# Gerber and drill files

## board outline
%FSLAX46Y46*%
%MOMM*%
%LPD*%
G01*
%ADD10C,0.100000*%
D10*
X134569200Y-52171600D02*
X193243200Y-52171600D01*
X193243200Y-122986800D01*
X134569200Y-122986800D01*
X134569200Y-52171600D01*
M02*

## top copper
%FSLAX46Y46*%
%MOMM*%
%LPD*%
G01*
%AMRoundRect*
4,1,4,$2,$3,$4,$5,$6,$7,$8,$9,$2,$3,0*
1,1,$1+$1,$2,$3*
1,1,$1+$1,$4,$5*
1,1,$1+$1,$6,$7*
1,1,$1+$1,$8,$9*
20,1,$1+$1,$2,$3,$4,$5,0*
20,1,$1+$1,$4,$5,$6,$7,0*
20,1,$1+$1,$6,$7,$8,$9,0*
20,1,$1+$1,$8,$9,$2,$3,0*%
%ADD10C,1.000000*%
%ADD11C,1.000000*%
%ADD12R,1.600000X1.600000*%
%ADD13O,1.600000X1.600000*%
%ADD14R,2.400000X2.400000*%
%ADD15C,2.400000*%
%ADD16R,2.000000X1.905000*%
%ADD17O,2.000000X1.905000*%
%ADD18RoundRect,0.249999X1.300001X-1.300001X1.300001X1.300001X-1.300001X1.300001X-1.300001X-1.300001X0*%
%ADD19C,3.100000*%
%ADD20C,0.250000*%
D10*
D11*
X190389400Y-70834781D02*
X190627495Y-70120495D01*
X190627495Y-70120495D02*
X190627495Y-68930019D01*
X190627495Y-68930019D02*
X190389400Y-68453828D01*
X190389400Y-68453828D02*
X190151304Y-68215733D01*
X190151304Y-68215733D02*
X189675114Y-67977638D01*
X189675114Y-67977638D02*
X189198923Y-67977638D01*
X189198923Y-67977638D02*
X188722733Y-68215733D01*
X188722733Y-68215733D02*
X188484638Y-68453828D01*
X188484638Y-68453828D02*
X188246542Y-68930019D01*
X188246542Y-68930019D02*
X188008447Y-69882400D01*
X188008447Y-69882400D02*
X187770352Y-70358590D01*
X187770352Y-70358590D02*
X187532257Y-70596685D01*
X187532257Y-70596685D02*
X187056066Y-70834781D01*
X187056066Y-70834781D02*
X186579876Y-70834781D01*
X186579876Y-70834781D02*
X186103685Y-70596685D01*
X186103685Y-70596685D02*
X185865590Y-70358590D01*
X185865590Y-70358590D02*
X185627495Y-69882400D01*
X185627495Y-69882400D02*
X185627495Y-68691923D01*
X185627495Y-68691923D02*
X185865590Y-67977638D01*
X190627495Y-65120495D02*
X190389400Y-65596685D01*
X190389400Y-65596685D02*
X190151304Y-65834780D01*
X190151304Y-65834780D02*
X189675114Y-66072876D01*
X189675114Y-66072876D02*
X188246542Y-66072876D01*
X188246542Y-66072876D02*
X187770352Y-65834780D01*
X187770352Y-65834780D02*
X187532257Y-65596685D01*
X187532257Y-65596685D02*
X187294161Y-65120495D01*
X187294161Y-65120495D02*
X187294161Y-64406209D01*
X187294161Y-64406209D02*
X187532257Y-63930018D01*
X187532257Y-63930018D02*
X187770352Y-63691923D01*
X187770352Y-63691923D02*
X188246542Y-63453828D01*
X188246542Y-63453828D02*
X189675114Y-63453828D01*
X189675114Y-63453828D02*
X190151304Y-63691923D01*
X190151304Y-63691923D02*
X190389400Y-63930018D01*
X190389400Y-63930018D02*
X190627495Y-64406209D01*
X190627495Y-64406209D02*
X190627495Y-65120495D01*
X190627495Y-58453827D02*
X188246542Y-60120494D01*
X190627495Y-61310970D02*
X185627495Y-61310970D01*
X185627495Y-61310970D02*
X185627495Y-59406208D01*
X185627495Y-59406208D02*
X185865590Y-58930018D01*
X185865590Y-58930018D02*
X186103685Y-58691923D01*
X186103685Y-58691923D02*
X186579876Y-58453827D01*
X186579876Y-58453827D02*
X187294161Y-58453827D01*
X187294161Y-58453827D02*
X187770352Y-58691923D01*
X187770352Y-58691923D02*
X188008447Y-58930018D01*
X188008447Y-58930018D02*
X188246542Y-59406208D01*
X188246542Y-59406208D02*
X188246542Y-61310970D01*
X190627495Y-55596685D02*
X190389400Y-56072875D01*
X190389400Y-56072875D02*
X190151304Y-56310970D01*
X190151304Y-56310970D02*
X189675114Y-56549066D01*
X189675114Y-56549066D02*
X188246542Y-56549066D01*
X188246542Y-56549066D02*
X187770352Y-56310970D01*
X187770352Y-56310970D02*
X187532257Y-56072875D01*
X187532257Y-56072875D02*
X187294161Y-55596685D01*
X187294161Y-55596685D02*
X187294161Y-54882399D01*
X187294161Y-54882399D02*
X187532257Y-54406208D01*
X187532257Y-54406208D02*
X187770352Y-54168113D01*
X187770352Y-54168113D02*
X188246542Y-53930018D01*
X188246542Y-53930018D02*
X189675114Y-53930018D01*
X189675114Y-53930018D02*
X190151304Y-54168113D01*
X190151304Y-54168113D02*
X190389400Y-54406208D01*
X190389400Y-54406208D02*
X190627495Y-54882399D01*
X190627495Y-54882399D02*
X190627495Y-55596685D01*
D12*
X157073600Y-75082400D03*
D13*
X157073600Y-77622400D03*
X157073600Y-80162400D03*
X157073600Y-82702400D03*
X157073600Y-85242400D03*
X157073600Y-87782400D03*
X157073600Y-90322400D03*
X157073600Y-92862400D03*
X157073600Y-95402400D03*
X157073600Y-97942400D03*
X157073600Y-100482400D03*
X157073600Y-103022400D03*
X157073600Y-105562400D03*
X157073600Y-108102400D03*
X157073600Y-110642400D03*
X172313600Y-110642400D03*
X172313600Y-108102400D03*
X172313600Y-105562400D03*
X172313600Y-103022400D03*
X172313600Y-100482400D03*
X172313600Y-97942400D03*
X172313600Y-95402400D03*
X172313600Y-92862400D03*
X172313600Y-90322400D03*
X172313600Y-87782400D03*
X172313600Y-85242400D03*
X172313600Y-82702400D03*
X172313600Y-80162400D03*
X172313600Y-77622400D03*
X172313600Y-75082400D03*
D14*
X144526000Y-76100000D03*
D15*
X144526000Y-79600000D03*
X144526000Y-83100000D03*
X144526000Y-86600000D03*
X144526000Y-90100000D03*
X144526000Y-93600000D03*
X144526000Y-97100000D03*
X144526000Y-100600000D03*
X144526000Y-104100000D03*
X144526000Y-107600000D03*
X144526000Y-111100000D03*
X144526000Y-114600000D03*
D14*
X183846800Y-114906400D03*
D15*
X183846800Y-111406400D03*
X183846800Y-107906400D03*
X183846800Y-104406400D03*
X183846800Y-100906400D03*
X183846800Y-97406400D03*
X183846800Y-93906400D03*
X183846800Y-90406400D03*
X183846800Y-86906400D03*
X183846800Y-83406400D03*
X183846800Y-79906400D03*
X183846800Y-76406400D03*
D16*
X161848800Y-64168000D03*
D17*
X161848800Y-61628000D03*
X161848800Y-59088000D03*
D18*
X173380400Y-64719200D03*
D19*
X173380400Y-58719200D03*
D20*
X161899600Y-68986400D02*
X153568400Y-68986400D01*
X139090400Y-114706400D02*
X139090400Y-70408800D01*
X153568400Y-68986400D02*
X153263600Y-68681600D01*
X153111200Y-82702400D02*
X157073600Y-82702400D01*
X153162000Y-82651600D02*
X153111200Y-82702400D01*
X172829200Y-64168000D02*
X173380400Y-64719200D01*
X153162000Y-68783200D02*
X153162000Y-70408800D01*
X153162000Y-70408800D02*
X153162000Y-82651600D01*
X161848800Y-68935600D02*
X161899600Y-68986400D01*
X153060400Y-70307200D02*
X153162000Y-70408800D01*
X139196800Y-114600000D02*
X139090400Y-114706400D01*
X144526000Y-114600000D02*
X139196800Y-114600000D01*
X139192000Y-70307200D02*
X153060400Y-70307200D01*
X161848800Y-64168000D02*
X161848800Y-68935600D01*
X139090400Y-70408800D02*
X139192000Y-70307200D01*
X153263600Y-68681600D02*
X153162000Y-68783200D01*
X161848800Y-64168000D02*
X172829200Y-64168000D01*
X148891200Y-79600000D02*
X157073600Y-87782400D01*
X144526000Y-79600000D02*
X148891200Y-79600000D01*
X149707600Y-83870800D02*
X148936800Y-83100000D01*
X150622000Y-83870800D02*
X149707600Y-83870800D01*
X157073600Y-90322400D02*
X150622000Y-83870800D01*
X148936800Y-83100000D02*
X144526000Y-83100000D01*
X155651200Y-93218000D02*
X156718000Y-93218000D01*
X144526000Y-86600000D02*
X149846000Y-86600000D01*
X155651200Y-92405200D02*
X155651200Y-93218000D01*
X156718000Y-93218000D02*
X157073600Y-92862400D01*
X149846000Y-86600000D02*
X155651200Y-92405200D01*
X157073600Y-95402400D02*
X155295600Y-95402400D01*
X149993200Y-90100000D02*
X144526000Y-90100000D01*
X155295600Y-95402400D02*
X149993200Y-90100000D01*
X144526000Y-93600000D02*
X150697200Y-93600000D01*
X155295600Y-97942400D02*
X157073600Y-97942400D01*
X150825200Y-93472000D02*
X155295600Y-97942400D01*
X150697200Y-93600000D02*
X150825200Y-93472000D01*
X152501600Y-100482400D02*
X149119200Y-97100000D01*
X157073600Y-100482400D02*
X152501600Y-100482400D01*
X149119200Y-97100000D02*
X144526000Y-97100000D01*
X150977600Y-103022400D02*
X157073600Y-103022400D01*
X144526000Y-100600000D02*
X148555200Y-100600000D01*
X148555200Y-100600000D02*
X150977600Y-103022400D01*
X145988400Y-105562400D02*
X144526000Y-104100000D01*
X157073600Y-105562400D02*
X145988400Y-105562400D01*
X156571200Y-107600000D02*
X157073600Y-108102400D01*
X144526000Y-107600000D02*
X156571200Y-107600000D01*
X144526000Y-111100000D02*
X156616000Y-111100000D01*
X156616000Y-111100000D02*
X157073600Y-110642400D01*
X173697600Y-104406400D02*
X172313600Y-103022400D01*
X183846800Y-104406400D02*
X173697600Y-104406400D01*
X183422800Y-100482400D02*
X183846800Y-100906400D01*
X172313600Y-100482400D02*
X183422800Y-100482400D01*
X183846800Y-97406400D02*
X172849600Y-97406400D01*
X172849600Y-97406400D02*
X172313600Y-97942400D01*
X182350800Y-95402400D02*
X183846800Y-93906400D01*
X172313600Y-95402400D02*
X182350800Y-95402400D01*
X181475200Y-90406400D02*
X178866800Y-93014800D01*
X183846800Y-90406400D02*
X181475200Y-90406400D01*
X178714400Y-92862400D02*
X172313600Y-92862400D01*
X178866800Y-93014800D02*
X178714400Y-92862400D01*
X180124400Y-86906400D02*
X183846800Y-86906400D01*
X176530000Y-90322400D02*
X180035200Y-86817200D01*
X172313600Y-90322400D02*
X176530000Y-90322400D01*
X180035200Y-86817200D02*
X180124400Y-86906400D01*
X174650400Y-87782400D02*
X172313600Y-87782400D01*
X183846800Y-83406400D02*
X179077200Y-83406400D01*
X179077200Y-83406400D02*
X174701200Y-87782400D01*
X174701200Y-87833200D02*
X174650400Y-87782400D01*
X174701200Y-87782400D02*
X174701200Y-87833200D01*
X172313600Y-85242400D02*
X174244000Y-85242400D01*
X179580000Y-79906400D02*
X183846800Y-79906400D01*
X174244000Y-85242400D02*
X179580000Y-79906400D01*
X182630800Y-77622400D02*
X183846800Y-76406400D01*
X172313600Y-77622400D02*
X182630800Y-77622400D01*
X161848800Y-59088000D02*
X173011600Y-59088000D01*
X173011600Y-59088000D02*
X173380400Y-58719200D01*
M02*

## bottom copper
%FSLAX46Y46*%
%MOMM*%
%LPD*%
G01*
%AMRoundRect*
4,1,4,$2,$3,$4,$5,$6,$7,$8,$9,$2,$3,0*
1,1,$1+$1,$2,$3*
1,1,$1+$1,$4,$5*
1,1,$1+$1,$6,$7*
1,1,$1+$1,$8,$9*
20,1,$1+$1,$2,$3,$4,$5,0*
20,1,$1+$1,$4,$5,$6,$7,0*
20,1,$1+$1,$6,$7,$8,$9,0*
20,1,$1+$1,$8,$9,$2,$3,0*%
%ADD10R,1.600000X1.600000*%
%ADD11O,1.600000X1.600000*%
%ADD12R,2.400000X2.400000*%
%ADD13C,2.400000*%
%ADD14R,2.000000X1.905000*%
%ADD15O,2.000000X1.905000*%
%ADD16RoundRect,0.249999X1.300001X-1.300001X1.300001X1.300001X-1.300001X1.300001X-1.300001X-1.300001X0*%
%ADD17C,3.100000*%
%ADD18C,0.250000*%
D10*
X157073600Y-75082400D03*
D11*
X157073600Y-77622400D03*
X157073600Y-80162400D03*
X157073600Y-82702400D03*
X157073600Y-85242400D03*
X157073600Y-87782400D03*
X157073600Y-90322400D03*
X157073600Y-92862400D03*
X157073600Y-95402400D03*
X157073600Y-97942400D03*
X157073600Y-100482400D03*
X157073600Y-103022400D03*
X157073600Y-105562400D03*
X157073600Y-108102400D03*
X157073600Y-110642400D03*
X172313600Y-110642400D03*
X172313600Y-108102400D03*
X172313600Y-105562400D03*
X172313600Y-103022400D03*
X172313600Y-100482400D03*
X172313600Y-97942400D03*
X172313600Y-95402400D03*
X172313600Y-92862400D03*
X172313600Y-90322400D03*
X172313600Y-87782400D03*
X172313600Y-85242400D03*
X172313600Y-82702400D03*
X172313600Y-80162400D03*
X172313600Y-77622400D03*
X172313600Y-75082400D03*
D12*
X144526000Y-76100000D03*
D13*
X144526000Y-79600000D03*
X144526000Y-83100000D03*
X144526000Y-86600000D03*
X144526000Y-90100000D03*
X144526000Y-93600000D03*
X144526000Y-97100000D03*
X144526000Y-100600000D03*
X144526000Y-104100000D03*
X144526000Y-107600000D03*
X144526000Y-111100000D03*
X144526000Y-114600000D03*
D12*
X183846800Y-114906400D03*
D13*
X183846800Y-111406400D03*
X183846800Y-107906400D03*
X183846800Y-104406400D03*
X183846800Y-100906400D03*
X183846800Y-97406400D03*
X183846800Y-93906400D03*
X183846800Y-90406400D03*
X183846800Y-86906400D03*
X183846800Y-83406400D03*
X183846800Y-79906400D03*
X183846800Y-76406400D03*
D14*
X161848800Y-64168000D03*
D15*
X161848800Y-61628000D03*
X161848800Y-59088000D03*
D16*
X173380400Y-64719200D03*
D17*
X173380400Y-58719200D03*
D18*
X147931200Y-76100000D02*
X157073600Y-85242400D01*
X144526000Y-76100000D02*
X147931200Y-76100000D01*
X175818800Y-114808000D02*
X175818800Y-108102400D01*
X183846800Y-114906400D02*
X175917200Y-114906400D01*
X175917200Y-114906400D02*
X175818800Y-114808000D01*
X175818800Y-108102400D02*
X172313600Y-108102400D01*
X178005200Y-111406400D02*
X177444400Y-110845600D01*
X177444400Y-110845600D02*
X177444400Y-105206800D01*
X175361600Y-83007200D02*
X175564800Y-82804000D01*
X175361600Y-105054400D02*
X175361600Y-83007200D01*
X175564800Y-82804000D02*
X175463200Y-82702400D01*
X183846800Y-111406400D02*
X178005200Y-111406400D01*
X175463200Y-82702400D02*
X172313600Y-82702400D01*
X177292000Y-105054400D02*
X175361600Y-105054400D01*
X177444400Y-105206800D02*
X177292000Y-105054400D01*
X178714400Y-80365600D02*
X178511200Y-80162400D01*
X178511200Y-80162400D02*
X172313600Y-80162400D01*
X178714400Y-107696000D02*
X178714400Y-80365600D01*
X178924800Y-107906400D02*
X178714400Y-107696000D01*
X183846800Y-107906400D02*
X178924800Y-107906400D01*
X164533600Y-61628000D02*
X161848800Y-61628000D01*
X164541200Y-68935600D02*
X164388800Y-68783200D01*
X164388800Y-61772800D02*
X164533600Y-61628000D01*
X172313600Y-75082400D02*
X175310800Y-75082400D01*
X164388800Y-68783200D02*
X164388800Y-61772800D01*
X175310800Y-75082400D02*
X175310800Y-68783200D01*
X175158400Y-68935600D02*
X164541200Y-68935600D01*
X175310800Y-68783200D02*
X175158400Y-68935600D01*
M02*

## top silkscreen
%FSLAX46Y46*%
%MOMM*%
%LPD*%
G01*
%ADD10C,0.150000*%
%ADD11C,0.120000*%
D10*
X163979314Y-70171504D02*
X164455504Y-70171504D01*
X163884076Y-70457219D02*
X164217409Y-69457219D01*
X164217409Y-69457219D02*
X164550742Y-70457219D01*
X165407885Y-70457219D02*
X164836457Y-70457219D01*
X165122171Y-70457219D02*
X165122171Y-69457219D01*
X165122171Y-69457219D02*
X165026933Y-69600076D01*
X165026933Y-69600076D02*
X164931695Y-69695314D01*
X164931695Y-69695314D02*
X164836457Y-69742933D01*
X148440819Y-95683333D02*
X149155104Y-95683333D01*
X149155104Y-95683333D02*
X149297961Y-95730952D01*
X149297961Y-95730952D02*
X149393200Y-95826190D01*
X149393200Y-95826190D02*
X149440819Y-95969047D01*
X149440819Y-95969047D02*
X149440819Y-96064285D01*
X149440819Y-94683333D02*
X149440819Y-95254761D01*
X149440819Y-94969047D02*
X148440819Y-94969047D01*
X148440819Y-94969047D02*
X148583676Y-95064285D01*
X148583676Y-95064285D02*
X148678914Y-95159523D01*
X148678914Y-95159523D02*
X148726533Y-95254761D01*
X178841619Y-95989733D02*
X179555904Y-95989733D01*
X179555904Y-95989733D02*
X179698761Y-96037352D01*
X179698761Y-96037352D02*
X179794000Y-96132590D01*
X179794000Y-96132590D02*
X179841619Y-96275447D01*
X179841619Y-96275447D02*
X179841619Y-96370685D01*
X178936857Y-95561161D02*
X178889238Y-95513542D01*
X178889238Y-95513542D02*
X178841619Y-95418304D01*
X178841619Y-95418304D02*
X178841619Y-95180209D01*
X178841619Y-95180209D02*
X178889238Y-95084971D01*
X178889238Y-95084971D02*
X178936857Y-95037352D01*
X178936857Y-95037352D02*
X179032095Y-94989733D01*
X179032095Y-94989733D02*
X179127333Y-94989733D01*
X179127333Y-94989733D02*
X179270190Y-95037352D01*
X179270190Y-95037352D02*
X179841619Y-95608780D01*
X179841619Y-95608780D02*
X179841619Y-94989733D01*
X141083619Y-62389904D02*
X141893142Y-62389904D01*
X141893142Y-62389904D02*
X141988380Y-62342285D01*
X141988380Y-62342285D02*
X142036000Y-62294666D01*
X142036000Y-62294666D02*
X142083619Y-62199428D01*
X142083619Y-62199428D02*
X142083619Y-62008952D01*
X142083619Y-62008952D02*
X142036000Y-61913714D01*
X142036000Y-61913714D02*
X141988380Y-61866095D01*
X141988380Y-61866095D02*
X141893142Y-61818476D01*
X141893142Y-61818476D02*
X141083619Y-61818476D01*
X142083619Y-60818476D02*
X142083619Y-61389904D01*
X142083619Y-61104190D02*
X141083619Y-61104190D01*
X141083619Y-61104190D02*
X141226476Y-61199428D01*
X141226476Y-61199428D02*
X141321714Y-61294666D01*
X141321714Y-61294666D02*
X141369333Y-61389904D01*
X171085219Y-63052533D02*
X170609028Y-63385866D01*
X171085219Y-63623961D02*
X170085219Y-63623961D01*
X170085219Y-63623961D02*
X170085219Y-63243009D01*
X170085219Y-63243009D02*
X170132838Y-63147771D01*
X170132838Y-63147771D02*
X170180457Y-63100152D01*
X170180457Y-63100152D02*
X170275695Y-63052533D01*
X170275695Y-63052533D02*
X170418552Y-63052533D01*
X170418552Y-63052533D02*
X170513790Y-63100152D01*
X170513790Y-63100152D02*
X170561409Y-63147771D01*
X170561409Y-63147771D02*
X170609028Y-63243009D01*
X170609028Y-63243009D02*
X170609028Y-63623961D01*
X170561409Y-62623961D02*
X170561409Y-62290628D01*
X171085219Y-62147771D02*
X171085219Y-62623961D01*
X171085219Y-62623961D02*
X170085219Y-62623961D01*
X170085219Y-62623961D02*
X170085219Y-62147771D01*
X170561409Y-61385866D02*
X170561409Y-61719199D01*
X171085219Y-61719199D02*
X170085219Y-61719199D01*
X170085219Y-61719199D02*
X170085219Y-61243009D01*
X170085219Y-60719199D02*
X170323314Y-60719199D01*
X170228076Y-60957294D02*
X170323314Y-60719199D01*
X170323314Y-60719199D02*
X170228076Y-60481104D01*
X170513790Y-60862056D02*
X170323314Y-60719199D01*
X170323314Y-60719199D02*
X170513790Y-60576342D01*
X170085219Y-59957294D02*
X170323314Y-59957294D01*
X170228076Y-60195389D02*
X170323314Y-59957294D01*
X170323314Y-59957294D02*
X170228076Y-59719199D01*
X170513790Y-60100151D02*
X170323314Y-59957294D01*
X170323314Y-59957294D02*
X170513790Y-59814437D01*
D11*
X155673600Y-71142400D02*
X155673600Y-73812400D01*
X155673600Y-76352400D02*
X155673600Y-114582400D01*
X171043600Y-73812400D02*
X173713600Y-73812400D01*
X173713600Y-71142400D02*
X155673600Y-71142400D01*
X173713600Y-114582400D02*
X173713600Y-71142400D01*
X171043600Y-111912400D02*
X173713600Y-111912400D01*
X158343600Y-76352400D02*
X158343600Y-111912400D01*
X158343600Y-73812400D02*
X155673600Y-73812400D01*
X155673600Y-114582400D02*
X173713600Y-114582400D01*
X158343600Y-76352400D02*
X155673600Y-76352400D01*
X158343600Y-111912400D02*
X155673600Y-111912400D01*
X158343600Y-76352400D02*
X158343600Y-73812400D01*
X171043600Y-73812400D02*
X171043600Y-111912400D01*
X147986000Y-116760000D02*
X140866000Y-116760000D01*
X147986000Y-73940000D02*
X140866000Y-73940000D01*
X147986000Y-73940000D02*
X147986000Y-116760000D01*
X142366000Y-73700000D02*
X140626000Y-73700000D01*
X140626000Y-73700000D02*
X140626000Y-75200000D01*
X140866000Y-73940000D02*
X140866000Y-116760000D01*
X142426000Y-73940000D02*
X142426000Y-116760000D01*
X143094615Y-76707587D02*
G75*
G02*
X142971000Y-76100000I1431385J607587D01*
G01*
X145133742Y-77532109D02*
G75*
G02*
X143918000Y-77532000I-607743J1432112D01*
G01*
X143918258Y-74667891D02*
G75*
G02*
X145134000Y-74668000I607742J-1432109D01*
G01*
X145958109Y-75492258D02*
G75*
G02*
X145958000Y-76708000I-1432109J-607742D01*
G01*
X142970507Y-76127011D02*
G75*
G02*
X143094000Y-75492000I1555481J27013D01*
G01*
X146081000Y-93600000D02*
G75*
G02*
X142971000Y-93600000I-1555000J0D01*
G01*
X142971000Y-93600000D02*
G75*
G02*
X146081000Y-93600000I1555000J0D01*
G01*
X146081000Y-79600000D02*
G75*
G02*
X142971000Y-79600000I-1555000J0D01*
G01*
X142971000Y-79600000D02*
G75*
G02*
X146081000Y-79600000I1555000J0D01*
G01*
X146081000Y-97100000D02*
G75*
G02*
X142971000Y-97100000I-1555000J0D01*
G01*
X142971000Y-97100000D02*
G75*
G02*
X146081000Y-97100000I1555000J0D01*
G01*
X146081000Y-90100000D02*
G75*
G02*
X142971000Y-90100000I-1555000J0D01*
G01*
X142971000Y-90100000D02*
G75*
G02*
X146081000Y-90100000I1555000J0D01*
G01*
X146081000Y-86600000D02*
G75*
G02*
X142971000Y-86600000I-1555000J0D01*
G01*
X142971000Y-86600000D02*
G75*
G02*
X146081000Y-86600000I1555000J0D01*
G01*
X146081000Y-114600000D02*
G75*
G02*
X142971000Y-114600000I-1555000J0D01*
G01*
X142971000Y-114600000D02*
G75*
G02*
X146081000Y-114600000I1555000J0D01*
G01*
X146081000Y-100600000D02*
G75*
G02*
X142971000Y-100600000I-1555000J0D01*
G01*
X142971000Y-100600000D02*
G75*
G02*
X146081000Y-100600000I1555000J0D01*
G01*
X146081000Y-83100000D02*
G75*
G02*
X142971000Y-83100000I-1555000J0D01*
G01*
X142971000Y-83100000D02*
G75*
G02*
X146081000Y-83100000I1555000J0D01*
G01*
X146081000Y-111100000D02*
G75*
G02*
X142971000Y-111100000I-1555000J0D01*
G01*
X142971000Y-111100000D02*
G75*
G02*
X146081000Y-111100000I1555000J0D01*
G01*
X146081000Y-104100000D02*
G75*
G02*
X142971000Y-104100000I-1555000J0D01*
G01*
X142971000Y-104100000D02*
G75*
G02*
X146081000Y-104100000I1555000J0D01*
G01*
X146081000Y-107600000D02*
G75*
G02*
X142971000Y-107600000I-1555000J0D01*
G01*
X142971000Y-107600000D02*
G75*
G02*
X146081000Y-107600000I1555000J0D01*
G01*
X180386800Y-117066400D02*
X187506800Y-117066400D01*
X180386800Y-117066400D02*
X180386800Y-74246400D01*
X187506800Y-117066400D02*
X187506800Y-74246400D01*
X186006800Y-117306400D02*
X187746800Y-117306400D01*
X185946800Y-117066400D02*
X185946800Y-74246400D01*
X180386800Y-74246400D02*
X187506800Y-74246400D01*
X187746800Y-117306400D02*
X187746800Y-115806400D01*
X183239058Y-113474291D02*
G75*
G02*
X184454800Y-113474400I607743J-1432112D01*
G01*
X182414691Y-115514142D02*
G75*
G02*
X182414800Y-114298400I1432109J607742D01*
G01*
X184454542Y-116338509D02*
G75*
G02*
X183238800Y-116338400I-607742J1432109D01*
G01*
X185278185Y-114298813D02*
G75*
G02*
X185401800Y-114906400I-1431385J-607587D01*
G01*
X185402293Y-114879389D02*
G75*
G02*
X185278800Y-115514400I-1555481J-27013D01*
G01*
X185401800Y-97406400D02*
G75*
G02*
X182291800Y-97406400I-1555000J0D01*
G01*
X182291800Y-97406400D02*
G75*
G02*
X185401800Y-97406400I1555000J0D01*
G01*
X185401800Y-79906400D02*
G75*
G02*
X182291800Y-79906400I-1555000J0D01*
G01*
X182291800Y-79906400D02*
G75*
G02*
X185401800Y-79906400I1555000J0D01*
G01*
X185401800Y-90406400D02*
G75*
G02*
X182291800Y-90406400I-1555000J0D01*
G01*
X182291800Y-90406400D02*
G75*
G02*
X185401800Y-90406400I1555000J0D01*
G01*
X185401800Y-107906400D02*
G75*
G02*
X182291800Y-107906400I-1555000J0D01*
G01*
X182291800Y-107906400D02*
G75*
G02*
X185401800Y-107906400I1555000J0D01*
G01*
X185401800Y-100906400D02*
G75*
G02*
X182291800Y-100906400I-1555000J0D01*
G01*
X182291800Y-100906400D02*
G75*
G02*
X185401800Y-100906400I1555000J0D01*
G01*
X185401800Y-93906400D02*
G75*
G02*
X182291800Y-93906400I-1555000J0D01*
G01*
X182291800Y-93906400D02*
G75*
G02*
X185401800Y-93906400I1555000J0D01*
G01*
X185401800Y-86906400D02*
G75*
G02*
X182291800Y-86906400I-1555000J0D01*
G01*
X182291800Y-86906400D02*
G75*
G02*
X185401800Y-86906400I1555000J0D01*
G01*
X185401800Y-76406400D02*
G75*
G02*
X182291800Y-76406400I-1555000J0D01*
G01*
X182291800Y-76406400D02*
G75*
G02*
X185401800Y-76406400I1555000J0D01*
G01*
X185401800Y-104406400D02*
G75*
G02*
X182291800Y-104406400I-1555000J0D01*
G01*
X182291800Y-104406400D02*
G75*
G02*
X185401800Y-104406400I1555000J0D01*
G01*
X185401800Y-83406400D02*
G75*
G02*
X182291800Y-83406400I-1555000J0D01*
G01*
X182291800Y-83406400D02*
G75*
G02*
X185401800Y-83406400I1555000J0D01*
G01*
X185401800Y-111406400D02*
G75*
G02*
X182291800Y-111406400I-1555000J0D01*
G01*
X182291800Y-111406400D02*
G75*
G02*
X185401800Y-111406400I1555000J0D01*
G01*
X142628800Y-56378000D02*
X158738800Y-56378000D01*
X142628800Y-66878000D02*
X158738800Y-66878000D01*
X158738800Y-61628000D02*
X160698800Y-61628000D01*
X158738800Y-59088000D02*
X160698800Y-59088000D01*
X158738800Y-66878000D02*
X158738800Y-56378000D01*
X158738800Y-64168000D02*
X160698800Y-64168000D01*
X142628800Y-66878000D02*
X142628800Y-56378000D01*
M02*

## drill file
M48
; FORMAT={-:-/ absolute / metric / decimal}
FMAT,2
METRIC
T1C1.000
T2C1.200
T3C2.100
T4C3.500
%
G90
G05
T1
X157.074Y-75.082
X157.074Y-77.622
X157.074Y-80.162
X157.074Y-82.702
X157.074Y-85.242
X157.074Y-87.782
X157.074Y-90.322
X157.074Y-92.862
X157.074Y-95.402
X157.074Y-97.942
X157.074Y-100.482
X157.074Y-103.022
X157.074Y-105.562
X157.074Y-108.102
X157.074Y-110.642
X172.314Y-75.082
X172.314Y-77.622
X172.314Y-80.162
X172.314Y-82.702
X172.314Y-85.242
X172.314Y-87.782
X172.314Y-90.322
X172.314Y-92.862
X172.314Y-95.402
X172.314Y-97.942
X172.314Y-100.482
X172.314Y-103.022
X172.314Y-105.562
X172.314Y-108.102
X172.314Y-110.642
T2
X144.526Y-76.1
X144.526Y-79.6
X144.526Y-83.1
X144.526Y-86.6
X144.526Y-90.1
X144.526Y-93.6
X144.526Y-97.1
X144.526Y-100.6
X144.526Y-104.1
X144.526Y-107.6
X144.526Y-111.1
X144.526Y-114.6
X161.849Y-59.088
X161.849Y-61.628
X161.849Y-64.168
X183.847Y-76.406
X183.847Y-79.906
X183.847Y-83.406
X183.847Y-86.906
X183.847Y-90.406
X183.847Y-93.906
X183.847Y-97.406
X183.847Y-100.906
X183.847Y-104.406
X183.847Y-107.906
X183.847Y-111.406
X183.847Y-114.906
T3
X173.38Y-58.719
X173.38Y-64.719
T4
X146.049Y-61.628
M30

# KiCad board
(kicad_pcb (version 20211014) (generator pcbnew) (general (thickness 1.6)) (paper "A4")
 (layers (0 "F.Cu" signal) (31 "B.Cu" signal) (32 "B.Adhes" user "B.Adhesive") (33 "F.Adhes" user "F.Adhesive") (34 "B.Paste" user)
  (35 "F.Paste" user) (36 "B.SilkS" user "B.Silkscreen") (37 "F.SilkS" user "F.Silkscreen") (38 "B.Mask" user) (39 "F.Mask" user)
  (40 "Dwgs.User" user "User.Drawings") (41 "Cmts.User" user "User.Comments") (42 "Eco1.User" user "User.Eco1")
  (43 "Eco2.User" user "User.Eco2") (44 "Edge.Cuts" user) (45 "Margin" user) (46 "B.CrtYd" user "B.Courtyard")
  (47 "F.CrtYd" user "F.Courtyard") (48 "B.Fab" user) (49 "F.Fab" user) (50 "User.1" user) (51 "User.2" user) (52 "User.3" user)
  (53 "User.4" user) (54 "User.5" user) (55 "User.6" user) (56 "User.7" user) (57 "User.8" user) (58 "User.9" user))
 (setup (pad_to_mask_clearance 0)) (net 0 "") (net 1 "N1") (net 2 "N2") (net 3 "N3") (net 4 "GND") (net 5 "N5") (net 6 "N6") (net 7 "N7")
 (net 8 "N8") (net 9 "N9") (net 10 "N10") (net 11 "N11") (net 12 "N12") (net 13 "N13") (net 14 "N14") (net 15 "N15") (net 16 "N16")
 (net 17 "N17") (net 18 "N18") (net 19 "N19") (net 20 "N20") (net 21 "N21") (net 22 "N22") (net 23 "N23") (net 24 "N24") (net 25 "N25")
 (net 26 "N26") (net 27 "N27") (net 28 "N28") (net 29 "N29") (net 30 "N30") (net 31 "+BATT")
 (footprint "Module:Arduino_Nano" (layer "F.Cu") (at 157.0736 75.0824)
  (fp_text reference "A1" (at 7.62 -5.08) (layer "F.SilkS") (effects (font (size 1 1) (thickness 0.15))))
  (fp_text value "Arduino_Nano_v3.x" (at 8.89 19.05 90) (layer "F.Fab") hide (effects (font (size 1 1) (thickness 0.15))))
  (fp_line (start -1.4 -3.94) (end -1.4 -1.27) (layer "F.SilkS") (width 0.12))
  (fp_line (start -1.4 1.27) (end -1.4 39.5) (layer "F.SilkS") (width 0.12))
  (fp_line (start 13.97 -1.27) (end 16.64 -1.27) (layer "F.SilkS") (width 0.12))
  (fp_line (start 16.64 -3.94) (end -1.4 -3.94) (layer "F.SilkS") (width 0.12))
  (fp_line (start 16.64 39.5) (end 16.64 -3.94) (layer "F.SilkS") (width 0.12))
  (fp_line (start 13.97 36.83) (end 16.64 36.83) (layer "F.SilkS") (width 0.12))
  (fp_line (start 1.27 1.27) (end 1.27 36.83) (layer "F.SilkS") (width 0.12))
  (fp_line (start 1.27 -1.27) (end -1.4 -1.27) (layer "F.SilkS") (width 0.12))
  (fp_line (start -1.4 39.5) (end 16.64 39.5) (layer "F.SilkS") (width 0.12))
  (fp_line (start 1.27 1.27) (end -1.4 1.27) (layer "F.SilkS") (width 0.12))
  (fp_line (start 1.27 36.83) (end -1.4 36.83) (layer "F.SilkS") (width 0.12))
  (fp_line (start 1.27 1.27) (end 1.27 -1.27) (layer "F.SilkS") (width 0.12))
  (fp_line (start 13.97 -1.27) (end 13.97 36.83) (layer "F.SilkS") (width 0.12))
  (pad "1" thru_hole rect (at 0 0) (size 1.6 1.6) (drill 1) (layers *.Cu *.Mask) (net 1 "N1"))
  (pad "2" thru_hole oval (at 0 2.54) (size 1.6 1.6) (drill 1) (layers *.Cu *.Mask) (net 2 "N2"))
  (pad "3" thru_hole oval (at 0 5.08) (size 1.6 1.6) (drill 1) (layers *.Cu *.Mask) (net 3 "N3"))
  (pad "4" thru_hole oval (at 0 7.62) (size 1.6 1.6) (drill 1) (layers *.Cu *.Mask) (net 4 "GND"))
  (pad "5" thru_hole oval (at 0 10.16) (size 1.6 1.6) (drill 1) (layers *.Cu *.Mask) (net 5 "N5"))
  (pad "6" thru_hole oval (at 0 12.7) (size 1.6 1.6) (drill 1) (layers *.Cu *.Mask) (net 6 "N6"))
  (pad "7" thru_hole oval (at 0 15.24) (size 1.6 1.6) (drill 1) (layers *.Cu *.Mask) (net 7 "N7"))
  (pad "8" thru_hole oval (at 0 17.78) (size 1.6 1.6) (drill 1) (layers *.Cu *.Mask) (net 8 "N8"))
  (pad "9" thru_hole oval (at 0 20.32) (size 1.6 1.6) (drill 1) (layers *.Cu *.Mask) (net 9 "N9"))
  (pad "10" thru_hole oval (at 0 22.86) (size 1.6 1.6) (drill 1) (layers *.Cu *.Mask) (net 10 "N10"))
  (pad "11" thru_hole oval (at 0 25.4) (size 1.6 1.6) (drill 1) (layers *.Cu *.Mask) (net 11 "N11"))
  (pad "12" thru_hole oval (at 0 27.94) (size 1.6 1.6) (drill 1) (layers *.Cu *.Mask) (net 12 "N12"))
  (pad "13" thru_hole oval (at 0 30.48) (size 1.6 1.6) (drill 1) (layers *.Cu *.Mask) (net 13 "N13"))
  (pad "14" thru_hole oval (at 0 33.02) (size 1.6 1.6) (drill 1) (layers *.Cu *.Mask) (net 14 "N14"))
  (pad "15" thru_hole oval (at 0 35.56) (size 1.6 1.6) (drill 1) (layers *.Cu *.Mask) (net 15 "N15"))
  (pad "16" thru_hole oval (at 15.24 35.56) (size 1.6 1.6) (drill 1) (layers *.Cu *.Mask) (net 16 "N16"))
  (pad "17" thru_hole oval (at 15.24 33.02) (size 1.6 1.6) (drill 1) (layers *.Cu *.Mask) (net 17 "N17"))
  (pad "18" thru_hole oval (at 15.24 30.48) (size 1.6 1.6) (drill 1) (layers *.Cu *.Mask) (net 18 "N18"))
  (pad "19" thru_hole oval (at 15.24 27.94) (size 1.6 1.6) (drill 1) (layers *.Cu *.Mask) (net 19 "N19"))
  (pad "20" thru_hole oval (at 15.24 25.4) (size 1.6 1.6) (drill 1) (layers *.Cu *.Mask) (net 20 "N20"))
  (pad "21" thru_hole oval (at 15.24 22.86) (size 1.6 1.6) (drill 1) (layers *.Cu *.Mask) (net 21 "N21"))
  (pad "22" thru_hole oval (at 15.24 20.32) (size 1.6 1.6) (drill 1) (layers *.Cu *.Mask) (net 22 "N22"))
  (pad "23" thru_hole oval (at 15.24 17.78) (size 1.6 1.6) (drill 1) (layers *.Cu *.Mask) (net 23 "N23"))
  (pad "24" thru_hole oval (at 15.24 15.24) (size 1.6 1.6) (drill 1) (layers *.Cu *.Mask) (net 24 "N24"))
  (pad "25" thru_hole oval (at 15.24 12.7) (size 1.6 1.6) (drill 1) (layers *.Cu *.Mask) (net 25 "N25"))
  (pad "26" thru_hole oval (at 15.24 10.16) (size 1.6 1.6) (drill 1) (layers *.Cu *.Mask) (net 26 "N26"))
  (pad "27" thru_hole oval (at 15.24 7.62) (size 1.6 1.6) (drill 1) (layers *.Cu *.Mask) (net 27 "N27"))
  (pad "28" thru_hole oval (at 15.24 5.08) (size 1.6 1.6) (drill 1) (layers *.Cu *.Mask) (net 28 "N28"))
  (pad "29" thru_hole oval (at 15.24 2.54) (size 1.6 1.6) (drill 1) (layers *.Cu *.Mask) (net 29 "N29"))
  (pad "30" thru_hole oval (at 15.24 0) (size 1.6 1.6) (drill 1) (layers *.Cu *.Mask) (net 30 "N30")))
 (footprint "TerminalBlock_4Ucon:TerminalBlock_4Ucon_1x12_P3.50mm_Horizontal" (layer "F.Cu") (at 144.526 76.1 -90)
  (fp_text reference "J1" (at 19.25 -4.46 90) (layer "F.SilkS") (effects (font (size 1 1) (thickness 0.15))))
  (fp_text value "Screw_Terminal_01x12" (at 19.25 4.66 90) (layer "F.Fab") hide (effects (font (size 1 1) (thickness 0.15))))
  (fp_line (start 40.66 -3.46) (end 40.66 3.66) (layer "F.SilkS") (width 0.12))
  (fp_line (start -2.16 -3.46) (end -2.16 3.66) (layer "F.SilkS") (width 0.12))
  (fp_line (start -2.16 -3.46) (end 40.66 -3.46) (layer "F.SilkS") (width 0.12))
  (fp_line (start -2.4 2.16) (end -2.4 3.9) (layer "F.SilkS") (width 0.12))
  (fp_line (start -2.4 3.9) (end -0.9 3.9) (layer "F.SilkS") (width 0.12))
  (fp_line (start -2.16 3.66) (end 40.66 3.66) (layer "F.SilkS") (width 0.12))
  (fp_line (start -2.16 2.1) (end 40.66 2.1) (layer "F.SilkS") (width 0.12))
  (fp_arc (start 0.607587 1.431385) (mid 0.310017 1.523783) (end 0 1.555) (layer "F.SilkS") (width 0.12))
  (fp_arc (start 1.432109 -0.607742) (mid 1.555727 0.00014) (end 1.432 0.608) (layer "F.SilkS") (width 0.12))
  (fp_arc (start -1.432109 0.607742) (mid -1.555727 -0.00014) (end -1.432 -0.608) (layer "F.SilkS") (width 0.12))
  (fp_arc (start -0.607742 -1.432109) (mid 0.00014 -1.555727) (end 0.608 -1.432) (layer "F.SilkS") (width 0.12))
  (fp_arc (start 0.027011 1.555493) (mid -0.296984 1.527118) (end -0.608 1.432) (layer "F.SilkS") (width 0.12))
  (fp_circle (center 17.5 0) (end 19.055 0) (layer "F.SilkS") (width 0.12) (fill none))
  (fp_circle (center 3.5 0) (end 5.055 0) (layer "F.SilkS") (width 0.12) (fill none))
  (fp_circle (center 21 0) (end 22.555 0) (layer "F.SilkS") (width 0.12) (fill none))
  (fp_circle (center 14 0) (end 15.555 0) (layer "F.SilkS") (width 0.12) (fill none))
  (fp_circle (center 10.5 0) (end 12.055 0) (layer "F.SilkS") (width 0.12) (fill none))
  (fp_circle (center 38.5 0) (end 40.055 0) (layer "F.SilkS") (width 0.12) (fill none))
  (fp_circle (center 24.5 0) (end 26.055 0) (layer "F.SilkS") (width 0.12) (fill none))
  (fp_circle (center 7 0) (end 8.555 0) (layer "F.SilkS") (width 0.12) (fill none))
  (fp_circle (center 35 0) (end 36.555 0) (layer "F.SilkS") (width 0.12) (fill none))
  (fp_circle (center 28 0) (end 29.555 0) (layer "F.SilkS") (width 0.12) (fill none))
  (fp_circle (center 31.5 0) (end 33.055 0) (layer "F.SilkS") (width 0.12) (fill none))
  (pad "1" thru_hole rect (at 0 0 270) (size 2.4 2.4) (drill 1.2) (layers *.Cu *.Mask) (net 5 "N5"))
  (pad "2" thru_hole circle (at 3.5 0 270) (size 2.4 2.4) (drill 1.2) (layers *.Cu *.Mask) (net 6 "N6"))
  (pad "3" thru_hole circle (at 7 0 270) (size 2.4 2.4) (drill 1.2) (layers *.Cu *.Mask) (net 7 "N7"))
  (pad "4" thru_hole circle (at 10.5 0 270) (size 2.4 2.4) (drill 1.2) (layers *.Cu *.Mask) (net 8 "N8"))
  (pad "5" thru_hole circle (at 14 0 270) (size 2.4 2.4) (drill 1.2) (layers *.Cu *.Mask) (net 9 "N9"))
  (pad "6" thru_hole circle (at 17.5 0 270) (size 2.4 2.4) (drill 1.2) (layers *.Cu *.Mask) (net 10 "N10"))
  (pad "7" thru_hole circle (at 21 0 270) (size 2.4 2.4) (drill 1.2) (layers *.Cu *.Mask) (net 11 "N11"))
  (pad "8" thru_hole circle (at 24.5 0 270) (size 2.4 2.4) (drill 1.2) (layers *.Cu *.Mask) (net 12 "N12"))
  (pad "9" thru_hole circle (at 28 0 270) (size 2.4 2.4) (drill 1.2) (layers *.Cu *.Mask) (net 13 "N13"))
  (pad "10" thru_hole circle (at 31.5 0 270) (size 2.4 2.4) (drill 1.2) (layers *.Cu *.Mask) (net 14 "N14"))
  (pad "11" thru_hole circle (at 35 0 270) (size 2.4 2.4) (drill 1.2) (layers *.Cu *.Mask) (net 15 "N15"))
  (pad "12" thru_hole circle (at 38.5 0 270) (size 2.4 2.4) (drill 1.2) (layers *.Cu *.Mask) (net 4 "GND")))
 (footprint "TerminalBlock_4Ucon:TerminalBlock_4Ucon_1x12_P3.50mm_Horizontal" (layer "F.Cu") (at 183.8468 114.9064 90)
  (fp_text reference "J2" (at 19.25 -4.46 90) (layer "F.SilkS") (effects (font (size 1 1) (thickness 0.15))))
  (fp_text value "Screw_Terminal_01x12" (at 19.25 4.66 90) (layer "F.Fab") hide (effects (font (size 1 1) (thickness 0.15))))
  (fp_line (start -2.16 -3.46) (end -2.16 3.66) (layer "F.SilkS") (width 0.12))
  (fp_line (start -2.16 -3.46) (end 40.66 -3.46) (layer "F.SilkS") (width 0.12))
  (fp_line (start -2.16 3.66) (end 40.66 3.66) (layer "F.SilkS") (width 0.12))
  (fp_line (start -2.4 2.16) (end -2.4 3.9) (layer "F.SilkS") (width 0.12))
  (fp_line (start -2.16 2.1) (end 40.66 2.1) (layer "F.SilkS") (width 0.12))
  (fp_line (start 40.66 -3.46) (end 40.66 3.66) (layer "F.SilkS") (width 0.12))
  (fp_line (start -2.4 3.9) (end -0.9 3.9) (layer "F.SilkS") (width 0.12))
  (fp_arc (start 1.432109 -0.607742) (mid 1.555727 0.00014) (end 1.432 0.608) (layer "F.SilkS") (width 0.12))
  (fp_arc (start -0.607742 -1.432109) (mid 0.00014 -1.555727) (end 0.608 -1.432) (layer "F.SilkS") (width 0.12))
  (fp_arc (start -1.432109 0.607742) (mid -1.555727 -0.00014) (end -1.432 -0.608) (layer "F.SilkS") (width 0.12))
  (fp_arc (start 0.607587 1.431385) (mid 0.310017 1.523783) (end 0 1.555) (layer "F.SilkS") (width 0.12))
  (fp_arc (start 0.027011 1.555493) (mid -0.296984 1.527118) (end -0.608 1.432) (layer "F.SilkS") (width 0.12))
  (fp_circle (center 17.5 0) (end 19.055 0) (layer "F.SilkS") (width 0.12) (fill none))
  (fp_circle (center 35 0) (end 36.555 0) (layer "F.SilkS") (width 0.12) (fill none))
  (fp_circle (center 24.5 0) (end 26.055 0) (layer "F.SilkS") (width 0.12) (fill none))
  (fp_circle (center 7 0) (end 8.555 0) (layer "F.SilkS") (width 0.12) (fill none))
  (fp_circle (center 14 0) (end 15.555 0) (layer "F.SilkS") (width 0.12) (fill none))
  (fp_circle (center 21 0) (end 22.555 0) (layer "F.SilkS") (width 0.12) (fill none))
  (fp_circle (center 28 0) (end 29.555 0) (layer "F.SilkS") (width 0.12) (fill none))
  (fp_circle (center 38.5 0) (end 40.055 0) (layer "F.SilkS") (width 0.12) (fill none))
  (fp_circle (center 10.5 0) (end 12.055 0) (layer "F.SilkS") (width 0.12) (fill none))
  (fp_circle (center 31.5 0) (end 33.055 0) (layer "F.SilkS") (width 0.12) (fill none))
  (fp_circle (center 3.5 0) (end 5.055 0) (layer "F.SilkS") (width 0.12) (fill none))
  (pad "1" thru_hole rect (at 0 0 90) (size 2.4 2.4) (drill 1.2) (layers *.Cu *.Mask) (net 17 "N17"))
  (pad "2" thru_hole circle (at 3.5 0 90) (size 2.4 2.4) (drill 1.2) (layers *.Cu *.Mask) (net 27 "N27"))
  (pad "3" thru_hole circle (at 7 0 90) (size 2.4 2.4) (drill 1.2) (layers *.Cu *.Mask) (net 28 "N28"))
  (pad "4" thru_hole circle (at 10.5 0 90) (size 2.4 2.4) (drill 1.2) (layers *.Cu *.Mask) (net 19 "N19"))
  (pad "5" thru_hole circle (at 14 0 90) (size 2.4 2.4) (drill 1.2) (layers *.Cu *.Mask) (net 20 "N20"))
  (pad "6" thru_hole circle (at 17.5 0 90) (size 2.4 2.4) (drill 1.2) (layers *.Cu *.Mask) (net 21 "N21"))
  (pad "7" thru_hole circle (at 21 0 90) (size 2.4 2.4) (drill 1.2) (layers *.Cu *.Mask) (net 22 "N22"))
  (pad "8" thru_hole circle (at 24.5 0 90) (size 2.4 2.4) (drill 1.2) (layers *.Cu *.Mask) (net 23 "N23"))
  (pad "9" thru_hole circle (at 28 0 90) (size 2.4 2.4) (drill 1.2) (layers *.Cu *.Mask) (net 24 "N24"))
  (pad "10" thru_hole circle (at 31.5 0 90) (size 2.4 2.4) (drill 1.2) (layers *.Cu *.Mask) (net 25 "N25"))
  (pad "11" thru_hole circle (at 35 0 90) (size 2.4 2.4) (drill 1.2) (layers *.Cu *.Mask) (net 26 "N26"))
  (pad "12" thru_hole circle (at 38.5 0 90) (size 2.4 2.4) (drill 1.2) (layers *.Cu *.Mask) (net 29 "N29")))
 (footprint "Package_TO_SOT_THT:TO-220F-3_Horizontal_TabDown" (layer "F.Cu") (at 161.8488 64.168 90)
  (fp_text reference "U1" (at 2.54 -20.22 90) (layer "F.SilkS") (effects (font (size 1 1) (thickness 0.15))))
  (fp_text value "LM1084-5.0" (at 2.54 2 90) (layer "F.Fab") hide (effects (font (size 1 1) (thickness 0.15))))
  (fp_line (start 7.79 -19.22) (end 7.79 -3.11) (layer "F.SilkS") (width 0.12))
  (fp_line (start -2.71 -19.22) (end -2.71 -3.11) (layer "F.SilkS") (width 0.12))
  (fp_line (start 2.54 -3.11) (end 2.54 -1.15) (layer "F.SilkS") (width 0.12))
  (fp_line (start 5.08 -3.11) (end 5.08 -1.15) (layer "F.SilkS") (width 0.12))
  (fp_line (start -2.71 -3.11) (end 7.79 -3.11) (layer "F.SilkS") (width 0.12))
  (fp_line (start 0 -3.11) (end 0 -1.15) (layer "F.SilkS") (width 0.12))
  (fp_line (start -2.71 -19.22) (end 7.79 -19.22) (layer "F.SilkS") (width 0.12))
  (pad "" np_thru_hole oval (at 2.54 -15.8 90) (size 3.5 3.5) (drill 3.5) (layers *.Cu *.Mask))
  (pad "1" thru_hole rect (at 0 0 90) (size 1.905 2) (drill 1.2) (layers *.Cu *.Mask) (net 4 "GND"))
  (pad "2" thru_hole oval (at 2.54 0 90) (size 1.905 2) (drill 1.2) (layers *.Cu *.Mask) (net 30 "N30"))
  (pad "3" thru_hole oval (at 5.08 0 90) (size 1.905 2) (drill 1.2) (layers *.Cu *.Mask) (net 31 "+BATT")))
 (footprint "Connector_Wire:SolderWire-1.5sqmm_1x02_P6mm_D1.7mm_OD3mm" (layer "F.Cu") (at 173.3804 64.7192 90)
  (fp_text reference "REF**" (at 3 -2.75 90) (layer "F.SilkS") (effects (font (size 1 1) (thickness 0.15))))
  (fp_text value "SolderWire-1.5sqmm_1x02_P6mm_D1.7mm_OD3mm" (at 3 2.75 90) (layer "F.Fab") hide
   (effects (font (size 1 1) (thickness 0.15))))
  (pad "1" thru_hole roundrect (at 0 0 90) (size 3.1 3.1) (drill 2.1) (layers *.Cu *.Mask) (roundrect_rratio 0.08064483871) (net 4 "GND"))
  (pad "2" thru_hole circle (at 6 0 90) (size 3.1 3.1) (drill 2.1) (layers *.Cu *.Mask) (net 31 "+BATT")))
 (gr_rect (start 193.2432 122.9868) (end 134.5692 52.1716) (layer "Edge.Cuts") (width 0.1) (fill none))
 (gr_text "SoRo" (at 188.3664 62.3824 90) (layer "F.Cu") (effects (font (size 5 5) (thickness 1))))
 (segment (start 161.8996 68.9864) (end 153.5684 68.9864) (width 0.25) (layer "F.Cu") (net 4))
 (segment (start 139.0904 114.7064) (end 139.0904 70.4088) (width 0.25) (layer "F.Cu") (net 4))
 (segment (start 153.5684 68.9864) (end 153.2636 68.6816) (width 0.25) (layer "F.Cu") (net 4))
 (segment (start 153.1112 82.7024) (end 157.0736 82.7024) (width 0.25) (layer "F.Cu") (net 4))
 (segment (start 153.162 82.6516) (end 153.1112 82.7024) (width 0.25) (layer "F.Cu") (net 4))
 (segment (start 172.8292 64.168) (end 173.3804 64.7192) (width 0.25) (layer "F.Cu") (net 4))
 (segment (start 153.162 68.7832) (end 153.162 70.4088) (width 0.25) (layer "F.Cu") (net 4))
 (segment (start 153.162 70.4088) (end 153.162 82.6516) (width 0.25) (layer "F.Cu") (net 4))
 (segment (start 161.8488 68.9356) (end 161.8996 68.9864) (width 0.25) (layer "F.Cu") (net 4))
 (segment (start 153.0604 70.3072) (end 153.162 70.4088) (width 0.25) (layer "F.Cu") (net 4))
 (segment (start 139.1968 114.6) (end 139.0904 114.7064) (width 0.25) (layer "F.Cu") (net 4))
 (segment (start 144.526 114.6) (end 139.1968 114.6) (width 0.25) (layer "F.Cu") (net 4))
 (segment (start 139.192 70.3072) (end 153.0604 70.3072) (width 0.25) (layer "F.Cu") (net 4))
 (segment (start 161.8488 64.168) (end 161.8488 68.9356) (width 0.25) (layer "F.Cu") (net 4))
 (segment (start 139.0904 70.4088) (end 139.192 70.3072) (width 0.25) (layer "F.Cu") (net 4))
 (segment (start 153.2636 68.6816) (end 153.162 68.7832) (width 0.25) (layer "F.Cu") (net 4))
 (segment (start 161.8488 64.168) (end 172.8292 64.168) (width 0.25) (layer "F.Cu") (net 4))
 (segment (start 147.9312 76.1) (end 157.0736 85.2424) (width 0.25) (layer "B.Cu") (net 5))
 (segment (start 144.526 76.1) (end 147.9312 76.1) (width 0.25) (layer "B.Cu") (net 5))
 (segment (start 148.8912 79.6) (end 157.0736 87.7824) (width 0.25) (layer "F.Cu") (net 6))
 (segment (start 144.526 79.6) (end 148.8912 79.6) (width 0.25) (layer "F.Cu") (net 6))
 (segment (start 149.7076 83.8708) (end 148.9368 83.1) (width 0.25) (layer "F.Cu") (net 7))
 (segment (start 150.622 83.8708) (end 149.7076 83.8708) (width 0.25) (layer "F.Cu") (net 7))
 (segment (start 157.0736 90.3224) (end 150.622 83.8708) (width 0.25) (layer "F.Cu") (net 7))
 (segment (start 148.9368 83.1) (end 144.526 83.1) (width 0.25) (layer "F.Cu") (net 7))
 (segment (start 155.6512 93.218) (end 156.718 93.218) (width 0.25) (layer "F.Cu") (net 8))
 (segment (start 144.526 86.6) (end 149.846 86.6) (width 0.25) (layer "F.Cu") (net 8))
 (segment (start 155.6512 92.4052) (end 155.6512 93.218) (width 0.25) (layer "F.Cu") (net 8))
 (segment (start 156.718 93.218) (end 157.0736 92.8624) (width 0.25) (layer "F.Cu") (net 8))
 (segment (start 149.846 86.6) (end 155.6512 92.4052) (width 0.25) (layer "F.Cu") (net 8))
 (segment (start 157.0736 95.4024) (end 155.2956 95.4024) (width 0.25) (layer "F.Cu") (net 9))
 (segment (start 149.9932 90.1) (end 144.526 90.1) (width 0.25) (layer "F.Cu") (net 9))
 (segment (start 155.2956 95.4024) (end 149.9932 90.1) (width 0.25) (layer "F.Cu") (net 9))
 (segment (start 144.526 93.6) (end 150.6972 93.6) (width 0.25) (layer "F.Cu") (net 10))
 (segment (start 155.2956 97.9424) (end 157.0736 97.9424) (width 0.25) (layer "F.Cu") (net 10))
 (segment (start 150.8252 93.472) (end 155.2956 97.9424) (width 0.25) (layer "F.Cu") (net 10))
 (segment (start 150.6972 93.6) (end 150.8252 93.472) (width 0.25) (layer "F.Cu") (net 10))
 (segment (start 152.5016 100.4824) (end 149.1192 97.1) (width 0.25) (layer "F.Cu") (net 11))
 (segment (start 157.0736 100.4824) (end 152.5016 100.4824) (width 0.25) (layer "F.Cu") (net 11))
 (segment (start 149.1192 97.1) (end 144.526 97.1) (width 0.25) (layer "F.Cu") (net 11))
 (segment (start 150.9776 103.0224) (end 157.0736 103.0224) (width 0.25) (layer "F.Cu") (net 12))
 (segment (start 144.526 100.6) (end 148.5552 100.6) (width 0.25) (layer "F.Cu") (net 12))
 (segment (start 148.5552 100.6) (end 150.9776 103.0224) (width 0.25) (layer "F.Cu") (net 12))
 (segment (start 145.9884 105.5624) (end 144.526 104.1) (width 0.25) (layer "F.Cu") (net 13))
 (segment (start 157.0736 105.5624) (end 145.9884 105.5624) (width 0.25) (layer "F.Cu") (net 13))
 (segment (start 156.5712 107.6) (end 157.0736 108.1024) (width 0.25) (layer "F.Cu") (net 14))
 (segment (start 144.526 107.6) (end 156.5712 107.6) (width 0.25) (layer "F.Cu") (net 14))
 (segment (start 144.526 111.1) (end 156.616 111.1) (width 0.25) (layer "F.Cu") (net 15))
 (segment (start 156.616 111.1) (end 157.0736 110.6424) (width 0.25) (layer "F.Cu") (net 15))
 (segment (start 175.8188 114.808) (end 175.8188 108.1024) (width 0.25) (layer "B.Cu") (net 17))
 (segment (start 183.8468 114.9064) (end 175.9172 114.9064) (width 0.25) (layer "B.Cu") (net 17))
 (segment (start 175.9172 114.9064) (end 175.8188 114.808) (width 0.25) (layer "B.Cu") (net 17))
 (segment (start 175.8188 108.1024) (end 172.3136 108.1024) (width 0.25) (layer "B.Cu") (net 17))
 (segment (start 173.6976 104.4064) (end 172.3136 103.0224) (width 0.25) (layer "F.Cu") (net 19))
 (segment (start 183.8468 104.4064) (end 173.6976 104.4064) (width 0.25) (layer "F.Cu") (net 19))
 (segment (start 183.4228 100.4824) (end 183.8468 100.9064) (width 0.25) (layer "F.Cu") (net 20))
 (segment (start 172.3136 100.4824) (end 183.4228 100.4824) (width 0.25) (layer "F.Cu") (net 20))
 (segment (start 183.8468 97.4064) (end 172.8496 97.4064) (width 0.25) (layer "F.Cu") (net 21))
 (segment (start 172.8496 97.4064) (end 172.3136 97.9424) (width 0.25) (layer "F.Cu") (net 21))
 (segment (start 182.3508 95.4024) (end 183.8468 93.9064) (width 0.25) (layer "F.Cu") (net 22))
 (segment (start 172.3136 95.4024) (end 182.3508 95.4024) (width 0.25) (layer "F.Cu") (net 22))
 (segment (start 181.4752 90.4064) (end 178.8668 93.0148) (width 0.25) (layer "F.Cu") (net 23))
 (segment (start 183.8468 90.4064) (end 181.4752 90.4064) (width 0.25) (layer "F.Cu") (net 23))
 (segment (start 178.7144 92.8624) (end 172.3136 92.8624) (width 0.25) (layer "F.Cu") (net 23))
 (segment (start 178.8668 93.0148) (end 178.7144 92.8624) (width 0.25) (layer "F.Cu") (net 23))
 (segment (start 180.1244 86.9064) (end 183.8468 86.9064) (width 0.25) (layer "F.Cu") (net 24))
 (segment (start 176.53 90.3224) (end 180.0352 86.8172) (width 0.25) (layer "F.Cu") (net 24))
 (segment (start 172.3136 90.3224) (end 176.53 90.3224) (width 0.25) (layer "F.Cu") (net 24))
 (segment (start 180.0352 86.8172) (end 180.1244 86.9064) (width 0.25) (layer "F.Cu") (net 24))
 (segment (start 174.6504 87.7824) (end 172.3136 87.7824) (width 0.25) (layer "F.Cu") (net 25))
 (segment (start 183.8468 83.4064) (end 179.0772 83.4064) (width 0.25) (layer "F.Cu") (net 25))
 (segment (start 179.0772 83.4064) (end 174.7012 87.7824) (width 0.25) (layer "F.Cu") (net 25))
 (segment (start 174.7012 87.8332) (end 174.6504 87.7824) (width 0.25) (layer "F.Cu") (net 25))
 (segment (start 174.7012 87.7824) (end 174.7012 87.8332) (width 0.25) (layer "F.Cu") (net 25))
 (segment (start 172.3136 85.2424) (end 174.244 85.2424) (width 0.25) (layer "F.Cu") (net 26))
 (segment (start 179.58 79.9064) (end 183.8468 79.9064) (width 0.25) (layer "F.Cu") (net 26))
 (segment (start 174.244 85.2424) (end 179.58 79.9064) (width 0.25) (layer "F.Cu") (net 26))
 (segment (start 178.0052 111.4064) (end 177.4444 110.8456) (width 0.25) (layer "B.Cu") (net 27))
 (segment (start 177.4444 110.8456) (end 177.4444 105.2068) (width 0.25) (layer "B.Cu") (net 27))
 (segment (start 175.3616 83.0072) (end 175.5648 82.804) (width 0.25) (layer "B.Cu") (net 27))
 (segment (start 175.3616 105.0544) (end 175.3616 83.0072) (width 0.25) (layer "B.Cu") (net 27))
 (segment (start 175.5648 82.804) (end 175.4632 82.7024) (width 0.25) (layer "B.Cu") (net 27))
 (segment (start 183.8468 111.4064) (end 178.0052 111.4064) (width 0.25) (layer "B.Cu") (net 27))
 (segment (start 175.4632 82.7024) (end 172.3136 82.7024) (width 0.25) (layer "B.Cu") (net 27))
 (segment (start 177.292 105.0544) (end 175.3616 105.0544) (width 0.25) (layer "B.Cu") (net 27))
 (segment (start 177.4444 105.2068) (end 177.292 105.0544) (width 0.25) (layer "B.Cu") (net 27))
 (segment (start 178.7144 80.3656) (end 178.5112 80.1624) (width 0.25) (layer "B.Cu") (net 28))
 (segment (start 178.5112 80.1624) (end 172.3136 80.1624) (width 0.25) (layer "B.Cu") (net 28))
 (segment (start 178.7144 107.696) (end 178.7144 80.3656) (width 0.25) (layer "B.Cu") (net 28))
 (segment (start 178.9248 107.9064) (end 178.7144 107.696) (width 0.25) (layer "B.Cu") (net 28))
 (segment (start 183.8468 107.9064) (end 178.9248 107.9064) (width 0.25) (layer "B.Cu") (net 28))
 (segment (start 182.6308 77.6224) (end 183.8468 76.4064) (width 0.25) (layer "F.Cu") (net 29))
 (segment (start 172.3136 77.6224) (end 182.6308 77.6224) (width 0.25) (layer "F.Cu") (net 29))
 (segment (start 164.5336 61.628) (end 161.8488 61.628) (width 0.25) (layer "B.Cu") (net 30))
 (segment (start 164.5412 68.9356) (end 164.3888 68.7832) (width 0.25) (layer "B.Cu") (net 30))
 (segment (start 164.3888 61.7728) (end 164.5336 61.628) (width 0.25) (layer "B.Cu") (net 30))
 (segment (start 172.3136 75.0824) (end 175.3108 75.0824) (width 0.25) (layer "B.Cu") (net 30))
 (segment (start 164.3888 68.7832) (end 164.3888 61.7728) (width 0.25) (layer "B.Cu") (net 30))
 (segment (start 175.3108 75.0824) (end 175.3108 68.7832) (width 0.25) (layer "B.Cu") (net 30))
 (segment (start 175.1584 68.9356) (end 164.5412 68.9356) (width 0.25) (layer "B.Cu") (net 30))
 (segment (start 175.3108 68.7832) (end 175.1584 68.9356) (width 0.25) (layer "B.Cu") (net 30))
 (segment (start 161.8488 59.088) (end 173.0116 59.088) (width 0.25) (layer "F.Cu") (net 31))
 (segment (start 173.0116 59.088) (end 173.3804 58.7192) (width 0.25) (layer "F.Cu") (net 31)))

